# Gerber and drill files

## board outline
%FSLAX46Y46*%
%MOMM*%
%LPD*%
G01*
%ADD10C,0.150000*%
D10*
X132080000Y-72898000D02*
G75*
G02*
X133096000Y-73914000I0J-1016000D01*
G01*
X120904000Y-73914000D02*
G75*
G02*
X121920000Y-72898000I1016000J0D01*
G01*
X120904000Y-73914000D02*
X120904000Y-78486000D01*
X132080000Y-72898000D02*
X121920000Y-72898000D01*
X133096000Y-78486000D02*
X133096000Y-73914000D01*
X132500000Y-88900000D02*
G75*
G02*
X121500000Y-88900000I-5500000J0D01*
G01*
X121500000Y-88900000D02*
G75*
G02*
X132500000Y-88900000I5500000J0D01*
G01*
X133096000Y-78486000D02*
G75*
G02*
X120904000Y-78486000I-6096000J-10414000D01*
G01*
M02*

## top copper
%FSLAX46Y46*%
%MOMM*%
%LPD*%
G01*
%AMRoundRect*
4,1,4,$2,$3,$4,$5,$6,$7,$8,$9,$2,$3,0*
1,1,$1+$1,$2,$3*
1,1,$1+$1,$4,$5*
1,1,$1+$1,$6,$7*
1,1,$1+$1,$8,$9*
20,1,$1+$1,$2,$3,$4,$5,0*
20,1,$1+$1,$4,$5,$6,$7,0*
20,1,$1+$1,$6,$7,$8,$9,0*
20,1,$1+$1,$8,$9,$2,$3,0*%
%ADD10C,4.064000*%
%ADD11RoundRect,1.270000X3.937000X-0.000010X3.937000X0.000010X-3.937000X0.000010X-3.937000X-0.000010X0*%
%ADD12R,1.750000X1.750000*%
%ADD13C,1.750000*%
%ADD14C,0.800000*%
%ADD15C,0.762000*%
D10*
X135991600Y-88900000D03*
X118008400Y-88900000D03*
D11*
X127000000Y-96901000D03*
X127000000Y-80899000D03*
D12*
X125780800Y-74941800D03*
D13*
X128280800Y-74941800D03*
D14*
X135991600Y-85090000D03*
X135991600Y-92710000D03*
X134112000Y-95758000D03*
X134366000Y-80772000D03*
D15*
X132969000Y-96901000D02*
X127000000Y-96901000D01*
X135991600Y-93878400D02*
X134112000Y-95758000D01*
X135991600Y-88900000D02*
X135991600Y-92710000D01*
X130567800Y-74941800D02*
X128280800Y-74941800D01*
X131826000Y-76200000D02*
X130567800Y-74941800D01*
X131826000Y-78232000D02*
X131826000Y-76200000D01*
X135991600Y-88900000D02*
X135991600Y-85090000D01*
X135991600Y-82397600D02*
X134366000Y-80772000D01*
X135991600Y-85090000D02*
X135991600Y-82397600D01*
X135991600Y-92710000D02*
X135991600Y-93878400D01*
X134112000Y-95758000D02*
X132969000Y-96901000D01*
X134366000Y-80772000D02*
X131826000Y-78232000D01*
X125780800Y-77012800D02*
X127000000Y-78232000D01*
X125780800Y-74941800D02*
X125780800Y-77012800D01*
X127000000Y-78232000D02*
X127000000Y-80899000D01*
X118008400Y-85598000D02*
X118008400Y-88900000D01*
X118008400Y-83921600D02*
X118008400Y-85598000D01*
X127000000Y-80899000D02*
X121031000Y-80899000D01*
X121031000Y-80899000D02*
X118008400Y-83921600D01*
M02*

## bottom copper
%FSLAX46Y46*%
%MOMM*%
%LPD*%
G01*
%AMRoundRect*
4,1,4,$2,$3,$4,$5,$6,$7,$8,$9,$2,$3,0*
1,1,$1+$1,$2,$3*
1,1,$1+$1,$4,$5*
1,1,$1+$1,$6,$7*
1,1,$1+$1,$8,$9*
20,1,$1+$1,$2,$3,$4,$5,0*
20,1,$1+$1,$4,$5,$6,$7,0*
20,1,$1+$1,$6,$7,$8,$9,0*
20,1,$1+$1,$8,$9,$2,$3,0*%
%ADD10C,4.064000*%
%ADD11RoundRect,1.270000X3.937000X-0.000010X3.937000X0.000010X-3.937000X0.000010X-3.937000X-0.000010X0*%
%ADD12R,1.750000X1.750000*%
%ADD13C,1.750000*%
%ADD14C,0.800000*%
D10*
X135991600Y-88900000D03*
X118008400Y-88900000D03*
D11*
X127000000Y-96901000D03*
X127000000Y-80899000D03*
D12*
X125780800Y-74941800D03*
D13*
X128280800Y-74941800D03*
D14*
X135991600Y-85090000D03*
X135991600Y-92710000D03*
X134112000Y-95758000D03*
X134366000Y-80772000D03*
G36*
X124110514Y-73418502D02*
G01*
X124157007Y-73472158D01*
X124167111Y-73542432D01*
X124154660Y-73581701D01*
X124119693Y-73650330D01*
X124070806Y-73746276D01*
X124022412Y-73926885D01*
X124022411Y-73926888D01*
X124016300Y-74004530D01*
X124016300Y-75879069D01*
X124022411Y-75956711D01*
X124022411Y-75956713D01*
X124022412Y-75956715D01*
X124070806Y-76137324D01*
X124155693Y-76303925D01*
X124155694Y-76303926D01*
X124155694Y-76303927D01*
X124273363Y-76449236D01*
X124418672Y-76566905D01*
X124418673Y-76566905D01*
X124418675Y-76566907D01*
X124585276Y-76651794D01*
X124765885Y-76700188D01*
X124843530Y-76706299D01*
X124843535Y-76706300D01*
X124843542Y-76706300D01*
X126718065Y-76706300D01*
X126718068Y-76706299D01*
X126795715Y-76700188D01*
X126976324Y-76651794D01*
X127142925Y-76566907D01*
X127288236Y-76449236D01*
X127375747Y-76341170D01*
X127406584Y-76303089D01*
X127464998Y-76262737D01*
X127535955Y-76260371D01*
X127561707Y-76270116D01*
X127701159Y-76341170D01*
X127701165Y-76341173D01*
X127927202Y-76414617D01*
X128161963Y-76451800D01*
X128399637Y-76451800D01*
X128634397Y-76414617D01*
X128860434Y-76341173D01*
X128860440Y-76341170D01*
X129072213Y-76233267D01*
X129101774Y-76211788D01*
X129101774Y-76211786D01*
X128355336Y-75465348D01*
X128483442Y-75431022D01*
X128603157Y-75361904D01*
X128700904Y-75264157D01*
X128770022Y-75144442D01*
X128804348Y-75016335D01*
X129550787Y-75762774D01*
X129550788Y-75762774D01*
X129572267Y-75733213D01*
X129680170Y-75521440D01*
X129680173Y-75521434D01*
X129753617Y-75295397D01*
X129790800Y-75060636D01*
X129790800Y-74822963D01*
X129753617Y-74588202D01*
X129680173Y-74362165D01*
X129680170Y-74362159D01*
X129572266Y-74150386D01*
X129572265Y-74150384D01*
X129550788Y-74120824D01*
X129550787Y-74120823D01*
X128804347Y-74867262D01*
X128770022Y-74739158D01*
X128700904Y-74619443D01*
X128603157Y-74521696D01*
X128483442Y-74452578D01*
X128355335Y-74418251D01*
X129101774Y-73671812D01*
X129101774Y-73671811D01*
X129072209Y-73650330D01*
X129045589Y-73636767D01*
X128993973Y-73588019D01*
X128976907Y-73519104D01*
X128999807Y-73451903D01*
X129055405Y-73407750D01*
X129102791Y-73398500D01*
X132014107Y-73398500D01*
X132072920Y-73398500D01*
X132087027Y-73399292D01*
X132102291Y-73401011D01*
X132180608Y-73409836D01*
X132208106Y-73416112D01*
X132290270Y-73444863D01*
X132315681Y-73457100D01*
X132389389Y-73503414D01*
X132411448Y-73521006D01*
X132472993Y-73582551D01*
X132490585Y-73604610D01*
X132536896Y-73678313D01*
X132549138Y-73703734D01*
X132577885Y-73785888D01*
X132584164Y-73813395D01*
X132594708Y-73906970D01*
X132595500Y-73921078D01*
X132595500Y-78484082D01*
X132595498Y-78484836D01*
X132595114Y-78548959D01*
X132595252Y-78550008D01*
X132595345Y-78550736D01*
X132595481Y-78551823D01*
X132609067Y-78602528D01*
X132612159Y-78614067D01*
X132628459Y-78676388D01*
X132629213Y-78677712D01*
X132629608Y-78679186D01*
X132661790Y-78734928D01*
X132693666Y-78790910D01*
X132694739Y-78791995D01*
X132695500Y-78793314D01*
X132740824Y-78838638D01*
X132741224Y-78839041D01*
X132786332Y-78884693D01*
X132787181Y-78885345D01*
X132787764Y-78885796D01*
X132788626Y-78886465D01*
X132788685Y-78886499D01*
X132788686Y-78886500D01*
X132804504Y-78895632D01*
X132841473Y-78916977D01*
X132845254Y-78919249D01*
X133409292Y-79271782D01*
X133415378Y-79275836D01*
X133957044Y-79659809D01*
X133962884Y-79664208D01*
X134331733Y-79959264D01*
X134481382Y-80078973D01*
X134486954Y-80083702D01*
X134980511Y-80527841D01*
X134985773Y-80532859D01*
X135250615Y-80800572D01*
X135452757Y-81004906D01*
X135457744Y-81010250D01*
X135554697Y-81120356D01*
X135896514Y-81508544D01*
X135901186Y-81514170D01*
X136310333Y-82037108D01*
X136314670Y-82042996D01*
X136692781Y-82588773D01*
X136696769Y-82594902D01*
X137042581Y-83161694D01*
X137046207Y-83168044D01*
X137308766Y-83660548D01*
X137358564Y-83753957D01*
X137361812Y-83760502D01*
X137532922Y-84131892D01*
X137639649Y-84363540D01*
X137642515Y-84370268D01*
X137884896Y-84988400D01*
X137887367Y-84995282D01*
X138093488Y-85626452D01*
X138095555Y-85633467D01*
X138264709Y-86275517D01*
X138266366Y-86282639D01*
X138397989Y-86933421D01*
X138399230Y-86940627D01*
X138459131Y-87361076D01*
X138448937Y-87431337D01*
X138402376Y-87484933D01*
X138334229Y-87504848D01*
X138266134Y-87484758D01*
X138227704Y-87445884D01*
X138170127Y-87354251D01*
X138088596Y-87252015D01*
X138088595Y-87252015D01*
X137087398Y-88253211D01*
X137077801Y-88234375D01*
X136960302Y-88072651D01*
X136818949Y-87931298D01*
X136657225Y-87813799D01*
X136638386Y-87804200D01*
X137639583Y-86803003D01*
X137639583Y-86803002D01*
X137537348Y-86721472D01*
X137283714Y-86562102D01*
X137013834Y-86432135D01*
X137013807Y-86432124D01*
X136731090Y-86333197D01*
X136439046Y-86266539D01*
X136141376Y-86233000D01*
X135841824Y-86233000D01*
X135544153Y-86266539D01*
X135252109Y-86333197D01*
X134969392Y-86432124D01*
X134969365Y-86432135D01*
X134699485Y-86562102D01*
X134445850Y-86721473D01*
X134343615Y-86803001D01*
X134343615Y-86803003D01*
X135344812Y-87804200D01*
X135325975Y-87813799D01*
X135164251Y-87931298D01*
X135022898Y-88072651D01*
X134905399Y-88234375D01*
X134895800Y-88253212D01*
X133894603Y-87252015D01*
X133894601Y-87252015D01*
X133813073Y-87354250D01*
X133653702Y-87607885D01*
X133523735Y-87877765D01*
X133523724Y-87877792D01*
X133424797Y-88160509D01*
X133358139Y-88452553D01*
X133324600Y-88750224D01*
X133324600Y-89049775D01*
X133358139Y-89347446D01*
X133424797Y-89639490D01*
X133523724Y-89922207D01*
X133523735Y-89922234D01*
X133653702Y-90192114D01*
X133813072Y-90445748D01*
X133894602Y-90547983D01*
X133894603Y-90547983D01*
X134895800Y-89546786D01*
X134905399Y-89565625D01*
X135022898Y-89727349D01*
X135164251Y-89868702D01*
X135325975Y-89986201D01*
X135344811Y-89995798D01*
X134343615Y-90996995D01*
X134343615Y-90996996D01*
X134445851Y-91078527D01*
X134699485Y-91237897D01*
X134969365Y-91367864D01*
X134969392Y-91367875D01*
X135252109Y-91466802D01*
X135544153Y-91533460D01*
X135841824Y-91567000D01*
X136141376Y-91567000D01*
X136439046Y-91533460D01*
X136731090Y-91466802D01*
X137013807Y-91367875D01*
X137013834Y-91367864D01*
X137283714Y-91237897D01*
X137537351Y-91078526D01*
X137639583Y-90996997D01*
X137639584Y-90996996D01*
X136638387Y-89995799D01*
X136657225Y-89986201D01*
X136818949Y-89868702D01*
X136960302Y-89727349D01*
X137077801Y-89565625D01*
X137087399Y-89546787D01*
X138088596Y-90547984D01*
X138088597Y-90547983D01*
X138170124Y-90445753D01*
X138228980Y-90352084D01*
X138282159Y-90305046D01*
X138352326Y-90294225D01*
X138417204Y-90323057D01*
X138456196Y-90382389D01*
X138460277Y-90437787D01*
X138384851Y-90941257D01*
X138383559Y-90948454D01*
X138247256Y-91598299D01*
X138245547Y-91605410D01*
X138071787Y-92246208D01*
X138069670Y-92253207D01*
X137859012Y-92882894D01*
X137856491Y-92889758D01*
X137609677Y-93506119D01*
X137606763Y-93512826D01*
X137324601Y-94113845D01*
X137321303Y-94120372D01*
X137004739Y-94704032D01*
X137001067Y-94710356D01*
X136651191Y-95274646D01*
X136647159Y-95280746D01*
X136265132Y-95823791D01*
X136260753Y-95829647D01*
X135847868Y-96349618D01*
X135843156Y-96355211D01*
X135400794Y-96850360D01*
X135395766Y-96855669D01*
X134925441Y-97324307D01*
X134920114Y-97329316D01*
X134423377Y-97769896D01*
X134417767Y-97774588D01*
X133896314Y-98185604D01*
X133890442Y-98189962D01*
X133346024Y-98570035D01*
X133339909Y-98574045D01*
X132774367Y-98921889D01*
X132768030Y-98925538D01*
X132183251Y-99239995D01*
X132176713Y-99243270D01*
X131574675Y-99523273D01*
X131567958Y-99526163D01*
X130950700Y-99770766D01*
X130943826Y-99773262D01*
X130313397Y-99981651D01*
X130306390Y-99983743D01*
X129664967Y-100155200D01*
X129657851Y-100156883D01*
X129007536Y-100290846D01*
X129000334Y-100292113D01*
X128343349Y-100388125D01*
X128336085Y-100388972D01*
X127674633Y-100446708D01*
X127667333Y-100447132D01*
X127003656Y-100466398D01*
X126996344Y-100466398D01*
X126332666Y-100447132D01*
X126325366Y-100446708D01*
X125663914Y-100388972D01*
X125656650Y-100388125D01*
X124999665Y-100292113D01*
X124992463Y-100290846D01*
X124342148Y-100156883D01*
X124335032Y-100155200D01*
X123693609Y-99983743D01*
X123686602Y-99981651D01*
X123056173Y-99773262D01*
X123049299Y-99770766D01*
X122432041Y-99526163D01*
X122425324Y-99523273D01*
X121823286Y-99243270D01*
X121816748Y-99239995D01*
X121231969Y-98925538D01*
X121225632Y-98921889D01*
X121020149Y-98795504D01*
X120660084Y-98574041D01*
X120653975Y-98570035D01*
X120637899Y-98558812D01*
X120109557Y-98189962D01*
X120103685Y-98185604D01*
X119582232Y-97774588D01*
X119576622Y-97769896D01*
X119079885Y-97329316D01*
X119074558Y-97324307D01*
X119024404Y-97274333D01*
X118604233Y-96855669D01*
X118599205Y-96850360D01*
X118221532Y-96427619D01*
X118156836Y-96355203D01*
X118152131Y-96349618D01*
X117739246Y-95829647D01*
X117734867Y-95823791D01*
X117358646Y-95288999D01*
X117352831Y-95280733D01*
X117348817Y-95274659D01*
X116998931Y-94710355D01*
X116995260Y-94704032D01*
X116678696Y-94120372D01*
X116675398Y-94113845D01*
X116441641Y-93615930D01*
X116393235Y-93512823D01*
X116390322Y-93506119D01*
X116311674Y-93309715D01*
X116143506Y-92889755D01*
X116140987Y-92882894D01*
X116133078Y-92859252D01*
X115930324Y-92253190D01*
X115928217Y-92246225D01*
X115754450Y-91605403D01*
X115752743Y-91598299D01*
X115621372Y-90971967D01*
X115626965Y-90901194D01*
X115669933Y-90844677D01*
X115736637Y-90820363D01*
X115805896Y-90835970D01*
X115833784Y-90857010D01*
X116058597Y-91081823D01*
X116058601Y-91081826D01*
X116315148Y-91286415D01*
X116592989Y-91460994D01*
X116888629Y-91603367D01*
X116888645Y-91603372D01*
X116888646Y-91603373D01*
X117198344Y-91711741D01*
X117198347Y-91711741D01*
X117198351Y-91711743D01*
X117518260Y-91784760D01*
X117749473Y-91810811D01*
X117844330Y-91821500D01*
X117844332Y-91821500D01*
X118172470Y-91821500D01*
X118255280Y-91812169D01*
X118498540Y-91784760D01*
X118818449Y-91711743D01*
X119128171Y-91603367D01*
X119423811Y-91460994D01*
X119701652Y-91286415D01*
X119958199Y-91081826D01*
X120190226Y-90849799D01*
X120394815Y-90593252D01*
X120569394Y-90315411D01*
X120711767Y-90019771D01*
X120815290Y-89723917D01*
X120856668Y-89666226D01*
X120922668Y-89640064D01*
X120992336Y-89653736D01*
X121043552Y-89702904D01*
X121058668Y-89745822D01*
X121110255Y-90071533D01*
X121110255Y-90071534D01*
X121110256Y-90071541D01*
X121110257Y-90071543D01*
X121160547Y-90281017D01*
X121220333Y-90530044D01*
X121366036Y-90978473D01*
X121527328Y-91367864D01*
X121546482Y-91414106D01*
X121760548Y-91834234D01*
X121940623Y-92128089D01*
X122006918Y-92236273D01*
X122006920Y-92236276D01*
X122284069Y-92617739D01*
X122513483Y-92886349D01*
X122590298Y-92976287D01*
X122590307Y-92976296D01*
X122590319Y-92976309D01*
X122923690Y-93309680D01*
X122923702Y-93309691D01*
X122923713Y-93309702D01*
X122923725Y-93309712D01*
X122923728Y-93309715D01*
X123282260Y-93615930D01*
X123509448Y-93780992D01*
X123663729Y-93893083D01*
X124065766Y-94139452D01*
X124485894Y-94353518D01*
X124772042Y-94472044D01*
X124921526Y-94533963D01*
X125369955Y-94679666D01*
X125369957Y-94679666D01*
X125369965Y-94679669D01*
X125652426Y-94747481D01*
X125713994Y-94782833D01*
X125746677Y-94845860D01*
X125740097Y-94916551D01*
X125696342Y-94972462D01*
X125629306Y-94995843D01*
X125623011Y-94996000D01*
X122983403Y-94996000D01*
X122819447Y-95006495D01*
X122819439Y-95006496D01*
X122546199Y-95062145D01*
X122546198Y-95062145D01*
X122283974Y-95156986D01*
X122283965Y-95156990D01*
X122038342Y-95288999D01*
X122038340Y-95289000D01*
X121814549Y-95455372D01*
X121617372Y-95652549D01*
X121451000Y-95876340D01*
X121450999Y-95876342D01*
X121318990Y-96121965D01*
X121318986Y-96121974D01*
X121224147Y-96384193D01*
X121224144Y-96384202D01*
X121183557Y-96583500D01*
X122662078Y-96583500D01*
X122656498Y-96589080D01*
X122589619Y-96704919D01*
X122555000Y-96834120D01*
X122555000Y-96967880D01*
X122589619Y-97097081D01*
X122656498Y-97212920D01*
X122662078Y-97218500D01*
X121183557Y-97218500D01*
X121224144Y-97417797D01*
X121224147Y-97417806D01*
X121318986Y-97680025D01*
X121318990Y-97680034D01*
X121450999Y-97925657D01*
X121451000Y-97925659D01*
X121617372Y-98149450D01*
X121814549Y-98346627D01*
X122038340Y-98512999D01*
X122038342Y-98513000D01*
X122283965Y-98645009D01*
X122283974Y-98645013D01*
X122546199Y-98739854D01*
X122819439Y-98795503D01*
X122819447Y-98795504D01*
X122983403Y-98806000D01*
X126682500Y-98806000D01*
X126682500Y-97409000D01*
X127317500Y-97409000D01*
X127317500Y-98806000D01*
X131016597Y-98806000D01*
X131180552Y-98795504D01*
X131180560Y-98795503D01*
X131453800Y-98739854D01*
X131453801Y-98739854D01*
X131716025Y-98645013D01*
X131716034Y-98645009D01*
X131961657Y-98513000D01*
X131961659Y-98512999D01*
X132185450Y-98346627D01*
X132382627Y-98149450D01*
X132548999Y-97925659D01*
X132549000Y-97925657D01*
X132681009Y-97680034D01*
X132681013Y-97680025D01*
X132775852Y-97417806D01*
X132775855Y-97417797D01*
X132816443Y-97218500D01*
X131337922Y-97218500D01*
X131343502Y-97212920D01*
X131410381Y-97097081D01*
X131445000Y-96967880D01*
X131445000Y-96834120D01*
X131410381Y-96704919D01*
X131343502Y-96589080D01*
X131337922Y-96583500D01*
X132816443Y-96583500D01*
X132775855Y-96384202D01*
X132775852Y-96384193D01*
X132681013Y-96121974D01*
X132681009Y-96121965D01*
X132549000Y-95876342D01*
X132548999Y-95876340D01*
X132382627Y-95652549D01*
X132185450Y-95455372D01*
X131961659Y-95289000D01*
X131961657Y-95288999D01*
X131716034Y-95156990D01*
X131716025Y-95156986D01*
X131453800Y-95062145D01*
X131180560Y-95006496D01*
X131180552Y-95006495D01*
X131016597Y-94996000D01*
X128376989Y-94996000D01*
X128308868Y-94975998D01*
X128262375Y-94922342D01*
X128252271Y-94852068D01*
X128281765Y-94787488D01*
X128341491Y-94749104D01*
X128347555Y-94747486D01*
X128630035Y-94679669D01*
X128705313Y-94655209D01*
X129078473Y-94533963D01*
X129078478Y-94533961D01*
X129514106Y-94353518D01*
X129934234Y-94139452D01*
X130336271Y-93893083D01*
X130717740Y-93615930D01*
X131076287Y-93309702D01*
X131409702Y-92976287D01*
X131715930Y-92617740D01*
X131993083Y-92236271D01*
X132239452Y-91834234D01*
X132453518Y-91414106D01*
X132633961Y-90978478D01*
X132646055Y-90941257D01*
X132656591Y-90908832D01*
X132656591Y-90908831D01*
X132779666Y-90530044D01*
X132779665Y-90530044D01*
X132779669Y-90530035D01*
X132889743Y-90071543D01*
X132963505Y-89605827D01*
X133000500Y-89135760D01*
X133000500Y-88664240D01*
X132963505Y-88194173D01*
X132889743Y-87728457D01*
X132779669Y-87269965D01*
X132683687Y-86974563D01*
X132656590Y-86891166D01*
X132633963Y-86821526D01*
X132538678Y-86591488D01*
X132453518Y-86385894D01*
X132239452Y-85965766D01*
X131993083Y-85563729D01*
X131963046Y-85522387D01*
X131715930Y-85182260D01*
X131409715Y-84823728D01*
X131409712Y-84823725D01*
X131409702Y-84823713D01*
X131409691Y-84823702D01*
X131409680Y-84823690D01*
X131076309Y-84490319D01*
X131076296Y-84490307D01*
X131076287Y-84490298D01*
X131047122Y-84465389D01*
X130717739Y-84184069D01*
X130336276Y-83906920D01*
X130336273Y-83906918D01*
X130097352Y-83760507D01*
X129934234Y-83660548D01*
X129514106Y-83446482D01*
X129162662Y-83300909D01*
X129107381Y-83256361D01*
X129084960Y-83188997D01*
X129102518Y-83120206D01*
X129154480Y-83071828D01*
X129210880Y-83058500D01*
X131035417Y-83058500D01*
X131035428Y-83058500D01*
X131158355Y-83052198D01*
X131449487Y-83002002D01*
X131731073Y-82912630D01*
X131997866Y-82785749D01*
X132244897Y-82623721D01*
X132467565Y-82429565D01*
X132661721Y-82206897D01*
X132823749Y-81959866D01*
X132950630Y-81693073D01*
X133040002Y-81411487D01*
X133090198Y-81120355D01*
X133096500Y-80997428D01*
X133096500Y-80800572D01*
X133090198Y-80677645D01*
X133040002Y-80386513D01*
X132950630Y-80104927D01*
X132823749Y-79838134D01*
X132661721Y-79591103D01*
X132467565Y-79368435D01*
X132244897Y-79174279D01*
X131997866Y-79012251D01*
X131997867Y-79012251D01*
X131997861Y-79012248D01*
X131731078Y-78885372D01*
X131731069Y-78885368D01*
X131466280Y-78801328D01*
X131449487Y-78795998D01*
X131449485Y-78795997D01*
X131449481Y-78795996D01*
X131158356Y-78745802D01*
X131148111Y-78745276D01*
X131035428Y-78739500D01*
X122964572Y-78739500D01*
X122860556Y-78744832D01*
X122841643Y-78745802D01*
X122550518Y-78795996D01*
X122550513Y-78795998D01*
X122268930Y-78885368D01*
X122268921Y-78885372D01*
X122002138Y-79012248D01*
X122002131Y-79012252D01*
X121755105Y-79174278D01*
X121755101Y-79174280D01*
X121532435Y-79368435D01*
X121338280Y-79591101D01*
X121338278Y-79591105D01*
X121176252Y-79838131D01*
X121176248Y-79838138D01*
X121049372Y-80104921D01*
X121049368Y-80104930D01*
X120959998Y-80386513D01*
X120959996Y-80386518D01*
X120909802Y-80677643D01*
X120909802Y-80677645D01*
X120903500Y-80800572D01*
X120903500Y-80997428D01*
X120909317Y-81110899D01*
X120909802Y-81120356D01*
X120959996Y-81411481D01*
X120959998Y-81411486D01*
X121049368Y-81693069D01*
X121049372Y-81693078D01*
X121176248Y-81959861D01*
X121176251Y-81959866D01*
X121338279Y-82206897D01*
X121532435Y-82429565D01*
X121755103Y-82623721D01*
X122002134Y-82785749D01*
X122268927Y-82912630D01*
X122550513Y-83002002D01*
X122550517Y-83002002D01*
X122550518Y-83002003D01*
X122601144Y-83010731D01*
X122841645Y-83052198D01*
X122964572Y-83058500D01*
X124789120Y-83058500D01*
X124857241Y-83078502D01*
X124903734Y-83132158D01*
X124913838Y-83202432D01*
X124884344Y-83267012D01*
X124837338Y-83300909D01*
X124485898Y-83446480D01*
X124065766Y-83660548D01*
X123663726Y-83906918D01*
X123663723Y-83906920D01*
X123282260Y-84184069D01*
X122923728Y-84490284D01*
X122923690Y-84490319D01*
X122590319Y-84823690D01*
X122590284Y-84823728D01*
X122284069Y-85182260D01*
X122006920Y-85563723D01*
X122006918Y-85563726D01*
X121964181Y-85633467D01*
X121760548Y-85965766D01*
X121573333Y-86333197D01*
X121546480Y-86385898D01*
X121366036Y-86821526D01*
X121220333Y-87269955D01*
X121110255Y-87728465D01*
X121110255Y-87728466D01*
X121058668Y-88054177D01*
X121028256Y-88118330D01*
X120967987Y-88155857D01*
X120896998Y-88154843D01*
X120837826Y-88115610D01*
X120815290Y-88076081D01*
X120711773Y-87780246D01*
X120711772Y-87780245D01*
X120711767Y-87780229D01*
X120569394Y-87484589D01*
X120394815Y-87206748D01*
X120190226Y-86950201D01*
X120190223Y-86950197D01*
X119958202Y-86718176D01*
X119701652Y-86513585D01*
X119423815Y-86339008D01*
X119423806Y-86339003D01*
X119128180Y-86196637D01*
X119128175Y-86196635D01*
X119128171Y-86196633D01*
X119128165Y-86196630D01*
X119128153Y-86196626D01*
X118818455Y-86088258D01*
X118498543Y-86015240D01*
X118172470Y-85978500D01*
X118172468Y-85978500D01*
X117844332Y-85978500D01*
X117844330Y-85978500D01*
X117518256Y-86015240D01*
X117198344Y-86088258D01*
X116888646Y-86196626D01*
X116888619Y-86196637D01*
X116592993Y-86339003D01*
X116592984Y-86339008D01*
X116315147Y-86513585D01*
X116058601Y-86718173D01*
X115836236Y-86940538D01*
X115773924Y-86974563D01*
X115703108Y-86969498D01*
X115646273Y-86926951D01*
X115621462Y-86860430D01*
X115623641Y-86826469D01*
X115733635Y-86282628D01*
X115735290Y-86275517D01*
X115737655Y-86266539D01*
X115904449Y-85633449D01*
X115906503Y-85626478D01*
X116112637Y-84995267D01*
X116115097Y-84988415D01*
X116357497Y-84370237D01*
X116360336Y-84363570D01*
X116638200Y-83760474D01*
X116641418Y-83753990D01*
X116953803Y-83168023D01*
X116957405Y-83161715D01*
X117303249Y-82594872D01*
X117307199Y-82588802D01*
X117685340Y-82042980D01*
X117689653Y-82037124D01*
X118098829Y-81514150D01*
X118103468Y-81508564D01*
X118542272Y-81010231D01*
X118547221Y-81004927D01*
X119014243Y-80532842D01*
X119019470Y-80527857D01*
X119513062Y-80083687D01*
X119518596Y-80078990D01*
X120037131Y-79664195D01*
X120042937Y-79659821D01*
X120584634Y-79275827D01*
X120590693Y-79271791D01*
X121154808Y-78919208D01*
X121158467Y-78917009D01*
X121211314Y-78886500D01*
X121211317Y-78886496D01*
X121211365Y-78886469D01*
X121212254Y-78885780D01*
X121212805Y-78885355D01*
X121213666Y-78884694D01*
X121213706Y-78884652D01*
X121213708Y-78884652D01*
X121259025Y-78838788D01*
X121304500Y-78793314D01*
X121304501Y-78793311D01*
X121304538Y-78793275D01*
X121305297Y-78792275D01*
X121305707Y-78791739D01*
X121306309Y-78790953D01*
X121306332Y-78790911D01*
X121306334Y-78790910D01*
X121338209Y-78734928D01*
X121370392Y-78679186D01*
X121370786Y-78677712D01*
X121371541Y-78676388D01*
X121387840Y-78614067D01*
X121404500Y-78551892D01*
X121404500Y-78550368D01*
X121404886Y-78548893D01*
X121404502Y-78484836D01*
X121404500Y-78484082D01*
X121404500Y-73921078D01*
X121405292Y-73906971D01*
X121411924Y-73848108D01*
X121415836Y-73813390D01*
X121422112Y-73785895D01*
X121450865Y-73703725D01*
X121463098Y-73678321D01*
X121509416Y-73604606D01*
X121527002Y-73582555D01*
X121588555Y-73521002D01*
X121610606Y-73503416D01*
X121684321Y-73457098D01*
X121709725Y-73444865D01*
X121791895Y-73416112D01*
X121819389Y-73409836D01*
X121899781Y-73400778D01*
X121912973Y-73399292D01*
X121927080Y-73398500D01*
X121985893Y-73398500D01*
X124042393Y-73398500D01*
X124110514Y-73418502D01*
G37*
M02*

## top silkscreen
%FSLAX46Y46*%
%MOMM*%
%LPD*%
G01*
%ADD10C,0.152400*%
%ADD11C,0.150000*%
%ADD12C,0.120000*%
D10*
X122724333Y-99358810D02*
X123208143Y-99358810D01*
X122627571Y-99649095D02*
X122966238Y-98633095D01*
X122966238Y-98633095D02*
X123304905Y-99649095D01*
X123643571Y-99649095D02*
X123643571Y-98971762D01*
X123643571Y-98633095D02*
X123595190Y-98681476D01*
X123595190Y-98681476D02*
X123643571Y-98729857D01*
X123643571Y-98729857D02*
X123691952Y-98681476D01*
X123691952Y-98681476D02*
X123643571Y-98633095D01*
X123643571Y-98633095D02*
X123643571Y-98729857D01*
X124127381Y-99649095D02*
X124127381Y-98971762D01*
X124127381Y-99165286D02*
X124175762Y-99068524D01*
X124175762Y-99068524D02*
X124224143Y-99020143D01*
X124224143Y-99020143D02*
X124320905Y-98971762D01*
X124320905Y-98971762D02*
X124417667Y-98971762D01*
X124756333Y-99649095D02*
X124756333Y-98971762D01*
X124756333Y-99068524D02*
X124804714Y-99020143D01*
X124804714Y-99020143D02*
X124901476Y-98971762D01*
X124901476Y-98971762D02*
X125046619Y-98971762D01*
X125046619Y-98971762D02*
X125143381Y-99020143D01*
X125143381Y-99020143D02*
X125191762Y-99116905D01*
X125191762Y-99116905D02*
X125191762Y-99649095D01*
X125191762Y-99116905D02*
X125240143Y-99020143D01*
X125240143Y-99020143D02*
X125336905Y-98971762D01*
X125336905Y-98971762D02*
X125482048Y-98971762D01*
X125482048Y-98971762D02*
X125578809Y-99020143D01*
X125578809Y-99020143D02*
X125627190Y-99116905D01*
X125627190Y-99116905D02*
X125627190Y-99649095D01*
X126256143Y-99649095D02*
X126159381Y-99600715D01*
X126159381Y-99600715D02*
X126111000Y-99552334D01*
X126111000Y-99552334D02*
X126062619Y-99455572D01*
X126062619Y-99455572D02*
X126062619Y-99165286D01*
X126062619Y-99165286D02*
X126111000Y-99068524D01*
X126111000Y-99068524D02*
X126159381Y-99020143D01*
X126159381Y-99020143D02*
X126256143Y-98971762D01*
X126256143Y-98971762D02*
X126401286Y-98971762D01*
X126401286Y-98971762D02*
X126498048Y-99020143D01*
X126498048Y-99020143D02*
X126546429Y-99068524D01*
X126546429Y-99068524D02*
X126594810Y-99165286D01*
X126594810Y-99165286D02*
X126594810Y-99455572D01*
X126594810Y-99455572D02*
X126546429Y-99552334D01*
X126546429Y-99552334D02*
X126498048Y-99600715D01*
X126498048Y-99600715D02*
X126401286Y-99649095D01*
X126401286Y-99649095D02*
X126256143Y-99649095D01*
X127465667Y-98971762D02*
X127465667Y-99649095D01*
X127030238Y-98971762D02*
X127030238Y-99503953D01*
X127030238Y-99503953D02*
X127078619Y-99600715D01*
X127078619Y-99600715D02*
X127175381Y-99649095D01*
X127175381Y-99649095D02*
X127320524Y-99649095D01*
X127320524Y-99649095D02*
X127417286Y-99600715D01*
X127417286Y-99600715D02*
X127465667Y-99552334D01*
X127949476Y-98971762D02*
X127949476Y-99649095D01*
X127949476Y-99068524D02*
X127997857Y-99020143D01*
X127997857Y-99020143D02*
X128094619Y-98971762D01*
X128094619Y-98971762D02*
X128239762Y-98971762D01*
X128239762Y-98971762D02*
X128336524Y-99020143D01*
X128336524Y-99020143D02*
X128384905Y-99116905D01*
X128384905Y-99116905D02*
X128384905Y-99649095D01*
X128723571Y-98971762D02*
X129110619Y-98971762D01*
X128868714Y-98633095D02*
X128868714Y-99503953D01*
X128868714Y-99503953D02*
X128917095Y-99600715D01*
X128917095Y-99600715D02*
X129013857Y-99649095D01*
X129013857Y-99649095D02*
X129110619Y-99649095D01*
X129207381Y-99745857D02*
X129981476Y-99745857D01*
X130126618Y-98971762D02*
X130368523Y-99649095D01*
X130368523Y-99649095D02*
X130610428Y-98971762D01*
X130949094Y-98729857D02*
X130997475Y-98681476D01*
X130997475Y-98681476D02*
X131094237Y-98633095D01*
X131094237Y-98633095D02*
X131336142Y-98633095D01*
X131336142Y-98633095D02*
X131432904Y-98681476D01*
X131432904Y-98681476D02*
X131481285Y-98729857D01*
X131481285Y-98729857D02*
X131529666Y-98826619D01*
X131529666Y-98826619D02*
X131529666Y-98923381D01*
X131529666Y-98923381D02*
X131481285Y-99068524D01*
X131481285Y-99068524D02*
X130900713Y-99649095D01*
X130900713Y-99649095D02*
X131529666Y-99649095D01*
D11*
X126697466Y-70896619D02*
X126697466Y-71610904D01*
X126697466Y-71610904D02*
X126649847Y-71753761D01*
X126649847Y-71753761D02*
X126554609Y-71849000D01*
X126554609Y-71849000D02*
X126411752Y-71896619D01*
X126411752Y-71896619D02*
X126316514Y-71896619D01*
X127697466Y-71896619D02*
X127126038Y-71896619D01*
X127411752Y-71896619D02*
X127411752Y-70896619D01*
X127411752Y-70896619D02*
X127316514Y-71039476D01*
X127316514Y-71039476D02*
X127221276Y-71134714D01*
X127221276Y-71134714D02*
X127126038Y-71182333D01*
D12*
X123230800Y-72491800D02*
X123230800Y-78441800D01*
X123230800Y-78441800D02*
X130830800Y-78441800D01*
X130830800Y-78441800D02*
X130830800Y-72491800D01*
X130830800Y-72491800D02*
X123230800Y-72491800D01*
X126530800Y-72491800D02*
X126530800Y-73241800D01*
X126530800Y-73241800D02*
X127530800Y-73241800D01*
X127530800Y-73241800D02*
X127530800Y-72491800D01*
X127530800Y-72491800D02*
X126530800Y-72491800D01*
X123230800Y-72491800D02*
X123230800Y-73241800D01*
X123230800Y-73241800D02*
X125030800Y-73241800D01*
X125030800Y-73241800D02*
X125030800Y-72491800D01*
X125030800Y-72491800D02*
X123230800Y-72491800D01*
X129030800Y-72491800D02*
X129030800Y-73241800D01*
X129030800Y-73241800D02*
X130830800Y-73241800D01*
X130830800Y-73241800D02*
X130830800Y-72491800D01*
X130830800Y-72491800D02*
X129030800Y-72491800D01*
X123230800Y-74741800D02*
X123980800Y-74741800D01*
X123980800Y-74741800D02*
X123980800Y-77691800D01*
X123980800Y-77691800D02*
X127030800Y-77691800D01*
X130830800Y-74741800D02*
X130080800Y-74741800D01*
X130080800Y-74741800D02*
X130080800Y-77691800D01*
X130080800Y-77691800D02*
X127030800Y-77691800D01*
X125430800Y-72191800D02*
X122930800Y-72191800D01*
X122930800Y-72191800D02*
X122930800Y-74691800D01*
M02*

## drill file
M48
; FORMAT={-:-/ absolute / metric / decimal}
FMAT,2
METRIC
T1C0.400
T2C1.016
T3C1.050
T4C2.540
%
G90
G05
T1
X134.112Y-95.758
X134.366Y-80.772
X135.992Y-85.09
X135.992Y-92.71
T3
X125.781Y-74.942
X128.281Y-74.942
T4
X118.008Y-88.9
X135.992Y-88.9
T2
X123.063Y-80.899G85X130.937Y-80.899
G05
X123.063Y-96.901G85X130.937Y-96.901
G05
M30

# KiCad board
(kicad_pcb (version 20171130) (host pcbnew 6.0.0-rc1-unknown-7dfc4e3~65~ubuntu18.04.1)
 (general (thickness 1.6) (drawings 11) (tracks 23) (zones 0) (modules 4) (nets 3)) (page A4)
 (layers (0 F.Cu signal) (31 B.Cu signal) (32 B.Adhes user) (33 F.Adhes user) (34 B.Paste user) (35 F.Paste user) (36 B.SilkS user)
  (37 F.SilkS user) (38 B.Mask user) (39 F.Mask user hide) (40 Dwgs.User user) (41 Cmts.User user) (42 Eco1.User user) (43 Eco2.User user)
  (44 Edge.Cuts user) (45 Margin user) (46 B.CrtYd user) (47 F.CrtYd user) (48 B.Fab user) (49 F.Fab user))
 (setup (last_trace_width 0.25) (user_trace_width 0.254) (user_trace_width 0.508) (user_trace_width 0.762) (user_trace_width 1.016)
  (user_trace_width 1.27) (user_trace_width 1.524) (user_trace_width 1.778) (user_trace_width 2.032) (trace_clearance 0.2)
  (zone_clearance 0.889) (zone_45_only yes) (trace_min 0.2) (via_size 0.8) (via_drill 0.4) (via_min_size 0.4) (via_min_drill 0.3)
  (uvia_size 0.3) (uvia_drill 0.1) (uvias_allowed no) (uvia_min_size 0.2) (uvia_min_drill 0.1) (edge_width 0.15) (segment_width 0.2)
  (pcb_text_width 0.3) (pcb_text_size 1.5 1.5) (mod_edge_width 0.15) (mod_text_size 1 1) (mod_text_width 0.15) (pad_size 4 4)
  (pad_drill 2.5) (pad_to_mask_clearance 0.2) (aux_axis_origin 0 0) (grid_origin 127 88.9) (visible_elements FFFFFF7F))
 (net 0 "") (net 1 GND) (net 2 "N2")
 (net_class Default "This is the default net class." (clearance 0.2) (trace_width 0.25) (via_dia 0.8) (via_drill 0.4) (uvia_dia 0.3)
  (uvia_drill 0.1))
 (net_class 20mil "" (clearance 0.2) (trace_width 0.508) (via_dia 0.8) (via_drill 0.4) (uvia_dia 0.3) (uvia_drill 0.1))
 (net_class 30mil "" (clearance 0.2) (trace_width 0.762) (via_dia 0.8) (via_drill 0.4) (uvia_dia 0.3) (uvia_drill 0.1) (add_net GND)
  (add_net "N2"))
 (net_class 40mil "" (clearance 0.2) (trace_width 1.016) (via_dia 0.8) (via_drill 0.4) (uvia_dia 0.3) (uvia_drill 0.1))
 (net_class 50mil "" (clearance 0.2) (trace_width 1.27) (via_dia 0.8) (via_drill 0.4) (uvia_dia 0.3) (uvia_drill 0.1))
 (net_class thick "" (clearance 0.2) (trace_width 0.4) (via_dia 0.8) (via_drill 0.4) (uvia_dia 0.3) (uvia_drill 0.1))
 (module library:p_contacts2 (layer F.Cu) (at 127 88.9)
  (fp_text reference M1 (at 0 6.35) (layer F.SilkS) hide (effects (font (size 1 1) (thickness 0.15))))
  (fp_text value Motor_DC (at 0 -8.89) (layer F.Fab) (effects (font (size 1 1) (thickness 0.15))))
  (pad 2 thru_hole circle (at 8.9916 0) (size 4.064 4.064) (drill 2.54) (layers *.Mask F.Cu) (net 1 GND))
  (pad 1 thru_hole circle (at -8.9916 0) (size 4.064 4.064) (drill 2.54) (layers *.Mask F.Cu) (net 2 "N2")))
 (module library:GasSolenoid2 (layer F.Cu) (at 127 88.9 90)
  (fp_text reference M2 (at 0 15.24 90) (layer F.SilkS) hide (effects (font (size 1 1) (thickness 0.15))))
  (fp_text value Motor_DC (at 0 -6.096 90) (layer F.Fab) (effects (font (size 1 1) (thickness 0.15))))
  (pad 2 thru_hole roundrect (at -8.001 0 90) (size 2.54 10.414) (drill oval 1.016 8.89) (layers *.Mask F.Cu) (roundrect_rratio 0.5)
   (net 1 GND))
  (pad 1 thru_hole roundrect (at 8.001 0 90) (size 2.54 10.414) (drill oval 1.016 8.89) (layers *.Mask F.Cu) (roundrect_rratio 0.5)
   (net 2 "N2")))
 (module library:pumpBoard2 (layer F.Cu) (at 127 88.9)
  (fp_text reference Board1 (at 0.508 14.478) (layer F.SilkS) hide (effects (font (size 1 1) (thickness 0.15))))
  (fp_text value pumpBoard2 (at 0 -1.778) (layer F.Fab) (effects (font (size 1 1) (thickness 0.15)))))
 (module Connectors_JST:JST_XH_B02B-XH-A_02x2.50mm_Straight (layer F.Cu) (at 125.7808 74.9418)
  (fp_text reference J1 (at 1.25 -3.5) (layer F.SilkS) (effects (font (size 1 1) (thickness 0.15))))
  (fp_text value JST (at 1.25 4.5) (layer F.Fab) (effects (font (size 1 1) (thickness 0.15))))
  (fp_line (start -2.55 -2.45) (end -2.55 3.5) (layer F.SilkS) (width 0.12))
  (fp_line (start -2.55 3.5) (end 5.05 3.5) (layer F.SilkS) (width 0.12))
  (fp_line (start 5.05 3.5) (end 5.05 -2.45) (layer F.SilkS) (width 0.12))
  (fp_line (start 5.05 -2.45) (end -2.55 -2.45) (layer F.SilkS) (width 0.12))
  (fp_line (start 0.75 -2.45) (end 0.75 -1.7) (layer F.SilkS) (width 0.12))
  (fp_line (start 0.75 -1.7) (end 1.75 -1.7) (layer F.SilkS) (width 0.12))
  (fp_line (start 1.75 -1.7) (end 1.75 -2.45) (layer F.SilkS) (width 0.12))
  (fp_line (start 1.75 -2.45) (end 0.75 -2.45) (layer F.SilkS) (width 0.12))
  (fp_line (start -2.55 -2.45) (end -2.55 -1.7) (layer F.SilkS) (width 0.12))
  (fp_line (start -2.55 -1.7) (end -0.75 -1.7) (layer F.SilkS) (width 0.12))
  (fp_line (start -0.75 -1.7) (end -0.75 -2.45) (layer F.SilkS) (width 0.12))
  (fp_line (start -0.75 -2.45) (end -2.55 -2.45) (layer F.SilkS) (width 0.12))
  (fp_line (start 3.25 -2.45) (end 3.25 -1.7) (layer F.SilkS) (width 0.12))
  (fp_line (start 3.25 -1.7) (end 5.05 -1.7) (layer F.SilkS) (width 0.12))
  (fp_line (start 5.05 -1.7) (end 5.05 -2.45) (layer F.SilkS) (width 0.12))
  (fp_line (start 5.05 -2.45) (end 3.25 -2.45) (layer F.SilkS) (width 0.12))
  (fp_line (start -2.55 -0.2) (end -1.8 -0.2) (layer F.SilkS) (width 0.12))
  (fp_line (start -1.8 -0.2) (end -1.8 2.75) (layer F.SilkS) (width 0.12))
  (fp_line (start -1.8 2.75) (end 1.25 2.75) (layer F.SilkS) (width 0.12))
  (fp_line (start 5.05 -0.2) (end 4.3 -0.2) (layer F.SilkS) (width 0.12))
  (fp_line (start 4.3 -0.2) (end 4.3 2.75) (layer F.SilkS) (width 0.12))
  (fp_line (start 4.3 2.75) (end 1.25 2.75) (layer F.SilkS) (width 0.12))
  (fp_line (start -0.35 -2.75) (end -2.85 -2.75) (layer F.SilkS) (width 0.12))
  (fp_line (start -2.85 -2.75) (end -2.85 -0.25) (layer F.SilkS) (width 0.12))
  (pad 1 thru_hole rect (at 0 0) (size 1.75 1.75) (drill 1.05) (layers *.Cu *.Mask) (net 2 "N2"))
  (pad 2 thru_hole circle (at 2.5 0) (size 1.75 1.75) (drill 1.05) (layers *.Cu *.Mask) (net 1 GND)))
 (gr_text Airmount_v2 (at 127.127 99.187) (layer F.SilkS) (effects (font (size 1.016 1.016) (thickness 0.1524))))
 (gr_arc (start 132.08 73.914) (end 133.096 73.914) (angle -90) (layer Edge.Cuts) (width 0.15))
 (gr_arc (start 121.92 73.914) (end 121.92 72.898) (angle -90) (layer Edge.Cuts) (width 0.15))
 (gr_line (start 120.904 73.914) (end 120.904 78.486) (layer Edge.Cuts) (width 0.15))
 (gr_line (start 132.08 72.898) (end 121.92 72.898) (layer Edge.Cuts) (width 0.15))
 (gr_line (start 133.096 78.486) (end 133.096 73.914) (layer Edge.Cuts) (width 0.15))
 (gr_circle (center 127 88.9) (end 132.5 88.9) (layer Edge.Cuts) (width 0.15))
 (gr_arc (start 127 88.9) (end 120.904 78.486) (angle -299.3135022) (layer Edge.Cuts) (width 0.15))
 (segment (start 132.969 96.901) (end 127 96.901) (width 0.762) (layer F.Cu) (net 1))
 (segment (start 135.9916 93.8784) (end 134.112 95.758) (width 0.762) (layer F.Cu) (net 1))
 (segment (start 135.9916 88.9) (end 135.9916 92.71) (width 0.762) (layer F.Cu) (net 1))
 (segment (start 130.5678 74.9418) (end 128.2808 74.9418) (width 0.762) (layer F.Cu) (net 1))
 (segment (start 131.826 76.2) (end 130.5678 74.9418) (width 0.762) (layer F.Cu) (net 1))
 (segment (start 131.826 78.232) (end 131.826 76.2) (width 0.762) (layer F.Cu) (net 1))
 (segment (start 135.9916 88.9) (end 135.9916 85.09) (width 0.762) (layer F.Cu) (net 1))
 (segment (start 135.9916 82.3976) (end 134.366 80.772) (width 0.762) (layer F.Cu) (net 1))
 (segment (start 135.9916 85.09) (end 135.9916 82.3976) (width 0.762) (layer F.Cu) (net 1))
 (via (at 135.9916 85.09) (size 0.8) (drill 0.4) (layers F.Cu B.Cu) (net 1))
 (segment (start 135.9916 92.71) (end 135.9916 93.8784) (width 0.762) (layer F.Cu) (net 1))
 (via (at 135.9916 92.71) (size 0.8) (drill 0.4) (layers F.Cu B.Cu) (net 1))
 (segment (start 134.112 95.758) (end 132.969 96.901) (width 0.762) (layer F.Cu) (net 1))
 (via (at 134.112 95.758) (size 0.8) (drill 0.4) (layers F.Cu B.Cu) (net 1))
 (segment (start 134.366 80.772) (end 131.826 78.232) (width 0.762) (layer F.Cu) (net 1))
 (via (at 134.366 80.772) (size 0.8) (drill 0.4) (layers F.Cu B.Cu) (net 1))
 (segment (start 125.7808 77.0128) (end 127 78.232) (width 0.762) (layer F.Cu) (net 2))
 (segment (start 125.7808 74.9418) (end 125.7808 77.0128) (width 0.762) (layer F.Cu) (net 2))
 (segment (start 127 78.232) (end 127 80.899) (width 0.762) (layer F.Cu) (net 2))
 (segment (start 118.0084 85.598) (end 118.0084 88.9) (width 0.762) (layer F.Cu) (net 2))
 (segment (start 118.0084 83.9216) (end 118.0084 85.598) (width 0.762) (layer F.Cu) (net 2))
 (segment (start 127 80.899) (end 121.031 80.899) (width 0.762) (layer F.Cu) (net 2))
 (segment (start 121.031 80.899) (end 118.0084 83.9216) (width 0.762) (layer F.Cu) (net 2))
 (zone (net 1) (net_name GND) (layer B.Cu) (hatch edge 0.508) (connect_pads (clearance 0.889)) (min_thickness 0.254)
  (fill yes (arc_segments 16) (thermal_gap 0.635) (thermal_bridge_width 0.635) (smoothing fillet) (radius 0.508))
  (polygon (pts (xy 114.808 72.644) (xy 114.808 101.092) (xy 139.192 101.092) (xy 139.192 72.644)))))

